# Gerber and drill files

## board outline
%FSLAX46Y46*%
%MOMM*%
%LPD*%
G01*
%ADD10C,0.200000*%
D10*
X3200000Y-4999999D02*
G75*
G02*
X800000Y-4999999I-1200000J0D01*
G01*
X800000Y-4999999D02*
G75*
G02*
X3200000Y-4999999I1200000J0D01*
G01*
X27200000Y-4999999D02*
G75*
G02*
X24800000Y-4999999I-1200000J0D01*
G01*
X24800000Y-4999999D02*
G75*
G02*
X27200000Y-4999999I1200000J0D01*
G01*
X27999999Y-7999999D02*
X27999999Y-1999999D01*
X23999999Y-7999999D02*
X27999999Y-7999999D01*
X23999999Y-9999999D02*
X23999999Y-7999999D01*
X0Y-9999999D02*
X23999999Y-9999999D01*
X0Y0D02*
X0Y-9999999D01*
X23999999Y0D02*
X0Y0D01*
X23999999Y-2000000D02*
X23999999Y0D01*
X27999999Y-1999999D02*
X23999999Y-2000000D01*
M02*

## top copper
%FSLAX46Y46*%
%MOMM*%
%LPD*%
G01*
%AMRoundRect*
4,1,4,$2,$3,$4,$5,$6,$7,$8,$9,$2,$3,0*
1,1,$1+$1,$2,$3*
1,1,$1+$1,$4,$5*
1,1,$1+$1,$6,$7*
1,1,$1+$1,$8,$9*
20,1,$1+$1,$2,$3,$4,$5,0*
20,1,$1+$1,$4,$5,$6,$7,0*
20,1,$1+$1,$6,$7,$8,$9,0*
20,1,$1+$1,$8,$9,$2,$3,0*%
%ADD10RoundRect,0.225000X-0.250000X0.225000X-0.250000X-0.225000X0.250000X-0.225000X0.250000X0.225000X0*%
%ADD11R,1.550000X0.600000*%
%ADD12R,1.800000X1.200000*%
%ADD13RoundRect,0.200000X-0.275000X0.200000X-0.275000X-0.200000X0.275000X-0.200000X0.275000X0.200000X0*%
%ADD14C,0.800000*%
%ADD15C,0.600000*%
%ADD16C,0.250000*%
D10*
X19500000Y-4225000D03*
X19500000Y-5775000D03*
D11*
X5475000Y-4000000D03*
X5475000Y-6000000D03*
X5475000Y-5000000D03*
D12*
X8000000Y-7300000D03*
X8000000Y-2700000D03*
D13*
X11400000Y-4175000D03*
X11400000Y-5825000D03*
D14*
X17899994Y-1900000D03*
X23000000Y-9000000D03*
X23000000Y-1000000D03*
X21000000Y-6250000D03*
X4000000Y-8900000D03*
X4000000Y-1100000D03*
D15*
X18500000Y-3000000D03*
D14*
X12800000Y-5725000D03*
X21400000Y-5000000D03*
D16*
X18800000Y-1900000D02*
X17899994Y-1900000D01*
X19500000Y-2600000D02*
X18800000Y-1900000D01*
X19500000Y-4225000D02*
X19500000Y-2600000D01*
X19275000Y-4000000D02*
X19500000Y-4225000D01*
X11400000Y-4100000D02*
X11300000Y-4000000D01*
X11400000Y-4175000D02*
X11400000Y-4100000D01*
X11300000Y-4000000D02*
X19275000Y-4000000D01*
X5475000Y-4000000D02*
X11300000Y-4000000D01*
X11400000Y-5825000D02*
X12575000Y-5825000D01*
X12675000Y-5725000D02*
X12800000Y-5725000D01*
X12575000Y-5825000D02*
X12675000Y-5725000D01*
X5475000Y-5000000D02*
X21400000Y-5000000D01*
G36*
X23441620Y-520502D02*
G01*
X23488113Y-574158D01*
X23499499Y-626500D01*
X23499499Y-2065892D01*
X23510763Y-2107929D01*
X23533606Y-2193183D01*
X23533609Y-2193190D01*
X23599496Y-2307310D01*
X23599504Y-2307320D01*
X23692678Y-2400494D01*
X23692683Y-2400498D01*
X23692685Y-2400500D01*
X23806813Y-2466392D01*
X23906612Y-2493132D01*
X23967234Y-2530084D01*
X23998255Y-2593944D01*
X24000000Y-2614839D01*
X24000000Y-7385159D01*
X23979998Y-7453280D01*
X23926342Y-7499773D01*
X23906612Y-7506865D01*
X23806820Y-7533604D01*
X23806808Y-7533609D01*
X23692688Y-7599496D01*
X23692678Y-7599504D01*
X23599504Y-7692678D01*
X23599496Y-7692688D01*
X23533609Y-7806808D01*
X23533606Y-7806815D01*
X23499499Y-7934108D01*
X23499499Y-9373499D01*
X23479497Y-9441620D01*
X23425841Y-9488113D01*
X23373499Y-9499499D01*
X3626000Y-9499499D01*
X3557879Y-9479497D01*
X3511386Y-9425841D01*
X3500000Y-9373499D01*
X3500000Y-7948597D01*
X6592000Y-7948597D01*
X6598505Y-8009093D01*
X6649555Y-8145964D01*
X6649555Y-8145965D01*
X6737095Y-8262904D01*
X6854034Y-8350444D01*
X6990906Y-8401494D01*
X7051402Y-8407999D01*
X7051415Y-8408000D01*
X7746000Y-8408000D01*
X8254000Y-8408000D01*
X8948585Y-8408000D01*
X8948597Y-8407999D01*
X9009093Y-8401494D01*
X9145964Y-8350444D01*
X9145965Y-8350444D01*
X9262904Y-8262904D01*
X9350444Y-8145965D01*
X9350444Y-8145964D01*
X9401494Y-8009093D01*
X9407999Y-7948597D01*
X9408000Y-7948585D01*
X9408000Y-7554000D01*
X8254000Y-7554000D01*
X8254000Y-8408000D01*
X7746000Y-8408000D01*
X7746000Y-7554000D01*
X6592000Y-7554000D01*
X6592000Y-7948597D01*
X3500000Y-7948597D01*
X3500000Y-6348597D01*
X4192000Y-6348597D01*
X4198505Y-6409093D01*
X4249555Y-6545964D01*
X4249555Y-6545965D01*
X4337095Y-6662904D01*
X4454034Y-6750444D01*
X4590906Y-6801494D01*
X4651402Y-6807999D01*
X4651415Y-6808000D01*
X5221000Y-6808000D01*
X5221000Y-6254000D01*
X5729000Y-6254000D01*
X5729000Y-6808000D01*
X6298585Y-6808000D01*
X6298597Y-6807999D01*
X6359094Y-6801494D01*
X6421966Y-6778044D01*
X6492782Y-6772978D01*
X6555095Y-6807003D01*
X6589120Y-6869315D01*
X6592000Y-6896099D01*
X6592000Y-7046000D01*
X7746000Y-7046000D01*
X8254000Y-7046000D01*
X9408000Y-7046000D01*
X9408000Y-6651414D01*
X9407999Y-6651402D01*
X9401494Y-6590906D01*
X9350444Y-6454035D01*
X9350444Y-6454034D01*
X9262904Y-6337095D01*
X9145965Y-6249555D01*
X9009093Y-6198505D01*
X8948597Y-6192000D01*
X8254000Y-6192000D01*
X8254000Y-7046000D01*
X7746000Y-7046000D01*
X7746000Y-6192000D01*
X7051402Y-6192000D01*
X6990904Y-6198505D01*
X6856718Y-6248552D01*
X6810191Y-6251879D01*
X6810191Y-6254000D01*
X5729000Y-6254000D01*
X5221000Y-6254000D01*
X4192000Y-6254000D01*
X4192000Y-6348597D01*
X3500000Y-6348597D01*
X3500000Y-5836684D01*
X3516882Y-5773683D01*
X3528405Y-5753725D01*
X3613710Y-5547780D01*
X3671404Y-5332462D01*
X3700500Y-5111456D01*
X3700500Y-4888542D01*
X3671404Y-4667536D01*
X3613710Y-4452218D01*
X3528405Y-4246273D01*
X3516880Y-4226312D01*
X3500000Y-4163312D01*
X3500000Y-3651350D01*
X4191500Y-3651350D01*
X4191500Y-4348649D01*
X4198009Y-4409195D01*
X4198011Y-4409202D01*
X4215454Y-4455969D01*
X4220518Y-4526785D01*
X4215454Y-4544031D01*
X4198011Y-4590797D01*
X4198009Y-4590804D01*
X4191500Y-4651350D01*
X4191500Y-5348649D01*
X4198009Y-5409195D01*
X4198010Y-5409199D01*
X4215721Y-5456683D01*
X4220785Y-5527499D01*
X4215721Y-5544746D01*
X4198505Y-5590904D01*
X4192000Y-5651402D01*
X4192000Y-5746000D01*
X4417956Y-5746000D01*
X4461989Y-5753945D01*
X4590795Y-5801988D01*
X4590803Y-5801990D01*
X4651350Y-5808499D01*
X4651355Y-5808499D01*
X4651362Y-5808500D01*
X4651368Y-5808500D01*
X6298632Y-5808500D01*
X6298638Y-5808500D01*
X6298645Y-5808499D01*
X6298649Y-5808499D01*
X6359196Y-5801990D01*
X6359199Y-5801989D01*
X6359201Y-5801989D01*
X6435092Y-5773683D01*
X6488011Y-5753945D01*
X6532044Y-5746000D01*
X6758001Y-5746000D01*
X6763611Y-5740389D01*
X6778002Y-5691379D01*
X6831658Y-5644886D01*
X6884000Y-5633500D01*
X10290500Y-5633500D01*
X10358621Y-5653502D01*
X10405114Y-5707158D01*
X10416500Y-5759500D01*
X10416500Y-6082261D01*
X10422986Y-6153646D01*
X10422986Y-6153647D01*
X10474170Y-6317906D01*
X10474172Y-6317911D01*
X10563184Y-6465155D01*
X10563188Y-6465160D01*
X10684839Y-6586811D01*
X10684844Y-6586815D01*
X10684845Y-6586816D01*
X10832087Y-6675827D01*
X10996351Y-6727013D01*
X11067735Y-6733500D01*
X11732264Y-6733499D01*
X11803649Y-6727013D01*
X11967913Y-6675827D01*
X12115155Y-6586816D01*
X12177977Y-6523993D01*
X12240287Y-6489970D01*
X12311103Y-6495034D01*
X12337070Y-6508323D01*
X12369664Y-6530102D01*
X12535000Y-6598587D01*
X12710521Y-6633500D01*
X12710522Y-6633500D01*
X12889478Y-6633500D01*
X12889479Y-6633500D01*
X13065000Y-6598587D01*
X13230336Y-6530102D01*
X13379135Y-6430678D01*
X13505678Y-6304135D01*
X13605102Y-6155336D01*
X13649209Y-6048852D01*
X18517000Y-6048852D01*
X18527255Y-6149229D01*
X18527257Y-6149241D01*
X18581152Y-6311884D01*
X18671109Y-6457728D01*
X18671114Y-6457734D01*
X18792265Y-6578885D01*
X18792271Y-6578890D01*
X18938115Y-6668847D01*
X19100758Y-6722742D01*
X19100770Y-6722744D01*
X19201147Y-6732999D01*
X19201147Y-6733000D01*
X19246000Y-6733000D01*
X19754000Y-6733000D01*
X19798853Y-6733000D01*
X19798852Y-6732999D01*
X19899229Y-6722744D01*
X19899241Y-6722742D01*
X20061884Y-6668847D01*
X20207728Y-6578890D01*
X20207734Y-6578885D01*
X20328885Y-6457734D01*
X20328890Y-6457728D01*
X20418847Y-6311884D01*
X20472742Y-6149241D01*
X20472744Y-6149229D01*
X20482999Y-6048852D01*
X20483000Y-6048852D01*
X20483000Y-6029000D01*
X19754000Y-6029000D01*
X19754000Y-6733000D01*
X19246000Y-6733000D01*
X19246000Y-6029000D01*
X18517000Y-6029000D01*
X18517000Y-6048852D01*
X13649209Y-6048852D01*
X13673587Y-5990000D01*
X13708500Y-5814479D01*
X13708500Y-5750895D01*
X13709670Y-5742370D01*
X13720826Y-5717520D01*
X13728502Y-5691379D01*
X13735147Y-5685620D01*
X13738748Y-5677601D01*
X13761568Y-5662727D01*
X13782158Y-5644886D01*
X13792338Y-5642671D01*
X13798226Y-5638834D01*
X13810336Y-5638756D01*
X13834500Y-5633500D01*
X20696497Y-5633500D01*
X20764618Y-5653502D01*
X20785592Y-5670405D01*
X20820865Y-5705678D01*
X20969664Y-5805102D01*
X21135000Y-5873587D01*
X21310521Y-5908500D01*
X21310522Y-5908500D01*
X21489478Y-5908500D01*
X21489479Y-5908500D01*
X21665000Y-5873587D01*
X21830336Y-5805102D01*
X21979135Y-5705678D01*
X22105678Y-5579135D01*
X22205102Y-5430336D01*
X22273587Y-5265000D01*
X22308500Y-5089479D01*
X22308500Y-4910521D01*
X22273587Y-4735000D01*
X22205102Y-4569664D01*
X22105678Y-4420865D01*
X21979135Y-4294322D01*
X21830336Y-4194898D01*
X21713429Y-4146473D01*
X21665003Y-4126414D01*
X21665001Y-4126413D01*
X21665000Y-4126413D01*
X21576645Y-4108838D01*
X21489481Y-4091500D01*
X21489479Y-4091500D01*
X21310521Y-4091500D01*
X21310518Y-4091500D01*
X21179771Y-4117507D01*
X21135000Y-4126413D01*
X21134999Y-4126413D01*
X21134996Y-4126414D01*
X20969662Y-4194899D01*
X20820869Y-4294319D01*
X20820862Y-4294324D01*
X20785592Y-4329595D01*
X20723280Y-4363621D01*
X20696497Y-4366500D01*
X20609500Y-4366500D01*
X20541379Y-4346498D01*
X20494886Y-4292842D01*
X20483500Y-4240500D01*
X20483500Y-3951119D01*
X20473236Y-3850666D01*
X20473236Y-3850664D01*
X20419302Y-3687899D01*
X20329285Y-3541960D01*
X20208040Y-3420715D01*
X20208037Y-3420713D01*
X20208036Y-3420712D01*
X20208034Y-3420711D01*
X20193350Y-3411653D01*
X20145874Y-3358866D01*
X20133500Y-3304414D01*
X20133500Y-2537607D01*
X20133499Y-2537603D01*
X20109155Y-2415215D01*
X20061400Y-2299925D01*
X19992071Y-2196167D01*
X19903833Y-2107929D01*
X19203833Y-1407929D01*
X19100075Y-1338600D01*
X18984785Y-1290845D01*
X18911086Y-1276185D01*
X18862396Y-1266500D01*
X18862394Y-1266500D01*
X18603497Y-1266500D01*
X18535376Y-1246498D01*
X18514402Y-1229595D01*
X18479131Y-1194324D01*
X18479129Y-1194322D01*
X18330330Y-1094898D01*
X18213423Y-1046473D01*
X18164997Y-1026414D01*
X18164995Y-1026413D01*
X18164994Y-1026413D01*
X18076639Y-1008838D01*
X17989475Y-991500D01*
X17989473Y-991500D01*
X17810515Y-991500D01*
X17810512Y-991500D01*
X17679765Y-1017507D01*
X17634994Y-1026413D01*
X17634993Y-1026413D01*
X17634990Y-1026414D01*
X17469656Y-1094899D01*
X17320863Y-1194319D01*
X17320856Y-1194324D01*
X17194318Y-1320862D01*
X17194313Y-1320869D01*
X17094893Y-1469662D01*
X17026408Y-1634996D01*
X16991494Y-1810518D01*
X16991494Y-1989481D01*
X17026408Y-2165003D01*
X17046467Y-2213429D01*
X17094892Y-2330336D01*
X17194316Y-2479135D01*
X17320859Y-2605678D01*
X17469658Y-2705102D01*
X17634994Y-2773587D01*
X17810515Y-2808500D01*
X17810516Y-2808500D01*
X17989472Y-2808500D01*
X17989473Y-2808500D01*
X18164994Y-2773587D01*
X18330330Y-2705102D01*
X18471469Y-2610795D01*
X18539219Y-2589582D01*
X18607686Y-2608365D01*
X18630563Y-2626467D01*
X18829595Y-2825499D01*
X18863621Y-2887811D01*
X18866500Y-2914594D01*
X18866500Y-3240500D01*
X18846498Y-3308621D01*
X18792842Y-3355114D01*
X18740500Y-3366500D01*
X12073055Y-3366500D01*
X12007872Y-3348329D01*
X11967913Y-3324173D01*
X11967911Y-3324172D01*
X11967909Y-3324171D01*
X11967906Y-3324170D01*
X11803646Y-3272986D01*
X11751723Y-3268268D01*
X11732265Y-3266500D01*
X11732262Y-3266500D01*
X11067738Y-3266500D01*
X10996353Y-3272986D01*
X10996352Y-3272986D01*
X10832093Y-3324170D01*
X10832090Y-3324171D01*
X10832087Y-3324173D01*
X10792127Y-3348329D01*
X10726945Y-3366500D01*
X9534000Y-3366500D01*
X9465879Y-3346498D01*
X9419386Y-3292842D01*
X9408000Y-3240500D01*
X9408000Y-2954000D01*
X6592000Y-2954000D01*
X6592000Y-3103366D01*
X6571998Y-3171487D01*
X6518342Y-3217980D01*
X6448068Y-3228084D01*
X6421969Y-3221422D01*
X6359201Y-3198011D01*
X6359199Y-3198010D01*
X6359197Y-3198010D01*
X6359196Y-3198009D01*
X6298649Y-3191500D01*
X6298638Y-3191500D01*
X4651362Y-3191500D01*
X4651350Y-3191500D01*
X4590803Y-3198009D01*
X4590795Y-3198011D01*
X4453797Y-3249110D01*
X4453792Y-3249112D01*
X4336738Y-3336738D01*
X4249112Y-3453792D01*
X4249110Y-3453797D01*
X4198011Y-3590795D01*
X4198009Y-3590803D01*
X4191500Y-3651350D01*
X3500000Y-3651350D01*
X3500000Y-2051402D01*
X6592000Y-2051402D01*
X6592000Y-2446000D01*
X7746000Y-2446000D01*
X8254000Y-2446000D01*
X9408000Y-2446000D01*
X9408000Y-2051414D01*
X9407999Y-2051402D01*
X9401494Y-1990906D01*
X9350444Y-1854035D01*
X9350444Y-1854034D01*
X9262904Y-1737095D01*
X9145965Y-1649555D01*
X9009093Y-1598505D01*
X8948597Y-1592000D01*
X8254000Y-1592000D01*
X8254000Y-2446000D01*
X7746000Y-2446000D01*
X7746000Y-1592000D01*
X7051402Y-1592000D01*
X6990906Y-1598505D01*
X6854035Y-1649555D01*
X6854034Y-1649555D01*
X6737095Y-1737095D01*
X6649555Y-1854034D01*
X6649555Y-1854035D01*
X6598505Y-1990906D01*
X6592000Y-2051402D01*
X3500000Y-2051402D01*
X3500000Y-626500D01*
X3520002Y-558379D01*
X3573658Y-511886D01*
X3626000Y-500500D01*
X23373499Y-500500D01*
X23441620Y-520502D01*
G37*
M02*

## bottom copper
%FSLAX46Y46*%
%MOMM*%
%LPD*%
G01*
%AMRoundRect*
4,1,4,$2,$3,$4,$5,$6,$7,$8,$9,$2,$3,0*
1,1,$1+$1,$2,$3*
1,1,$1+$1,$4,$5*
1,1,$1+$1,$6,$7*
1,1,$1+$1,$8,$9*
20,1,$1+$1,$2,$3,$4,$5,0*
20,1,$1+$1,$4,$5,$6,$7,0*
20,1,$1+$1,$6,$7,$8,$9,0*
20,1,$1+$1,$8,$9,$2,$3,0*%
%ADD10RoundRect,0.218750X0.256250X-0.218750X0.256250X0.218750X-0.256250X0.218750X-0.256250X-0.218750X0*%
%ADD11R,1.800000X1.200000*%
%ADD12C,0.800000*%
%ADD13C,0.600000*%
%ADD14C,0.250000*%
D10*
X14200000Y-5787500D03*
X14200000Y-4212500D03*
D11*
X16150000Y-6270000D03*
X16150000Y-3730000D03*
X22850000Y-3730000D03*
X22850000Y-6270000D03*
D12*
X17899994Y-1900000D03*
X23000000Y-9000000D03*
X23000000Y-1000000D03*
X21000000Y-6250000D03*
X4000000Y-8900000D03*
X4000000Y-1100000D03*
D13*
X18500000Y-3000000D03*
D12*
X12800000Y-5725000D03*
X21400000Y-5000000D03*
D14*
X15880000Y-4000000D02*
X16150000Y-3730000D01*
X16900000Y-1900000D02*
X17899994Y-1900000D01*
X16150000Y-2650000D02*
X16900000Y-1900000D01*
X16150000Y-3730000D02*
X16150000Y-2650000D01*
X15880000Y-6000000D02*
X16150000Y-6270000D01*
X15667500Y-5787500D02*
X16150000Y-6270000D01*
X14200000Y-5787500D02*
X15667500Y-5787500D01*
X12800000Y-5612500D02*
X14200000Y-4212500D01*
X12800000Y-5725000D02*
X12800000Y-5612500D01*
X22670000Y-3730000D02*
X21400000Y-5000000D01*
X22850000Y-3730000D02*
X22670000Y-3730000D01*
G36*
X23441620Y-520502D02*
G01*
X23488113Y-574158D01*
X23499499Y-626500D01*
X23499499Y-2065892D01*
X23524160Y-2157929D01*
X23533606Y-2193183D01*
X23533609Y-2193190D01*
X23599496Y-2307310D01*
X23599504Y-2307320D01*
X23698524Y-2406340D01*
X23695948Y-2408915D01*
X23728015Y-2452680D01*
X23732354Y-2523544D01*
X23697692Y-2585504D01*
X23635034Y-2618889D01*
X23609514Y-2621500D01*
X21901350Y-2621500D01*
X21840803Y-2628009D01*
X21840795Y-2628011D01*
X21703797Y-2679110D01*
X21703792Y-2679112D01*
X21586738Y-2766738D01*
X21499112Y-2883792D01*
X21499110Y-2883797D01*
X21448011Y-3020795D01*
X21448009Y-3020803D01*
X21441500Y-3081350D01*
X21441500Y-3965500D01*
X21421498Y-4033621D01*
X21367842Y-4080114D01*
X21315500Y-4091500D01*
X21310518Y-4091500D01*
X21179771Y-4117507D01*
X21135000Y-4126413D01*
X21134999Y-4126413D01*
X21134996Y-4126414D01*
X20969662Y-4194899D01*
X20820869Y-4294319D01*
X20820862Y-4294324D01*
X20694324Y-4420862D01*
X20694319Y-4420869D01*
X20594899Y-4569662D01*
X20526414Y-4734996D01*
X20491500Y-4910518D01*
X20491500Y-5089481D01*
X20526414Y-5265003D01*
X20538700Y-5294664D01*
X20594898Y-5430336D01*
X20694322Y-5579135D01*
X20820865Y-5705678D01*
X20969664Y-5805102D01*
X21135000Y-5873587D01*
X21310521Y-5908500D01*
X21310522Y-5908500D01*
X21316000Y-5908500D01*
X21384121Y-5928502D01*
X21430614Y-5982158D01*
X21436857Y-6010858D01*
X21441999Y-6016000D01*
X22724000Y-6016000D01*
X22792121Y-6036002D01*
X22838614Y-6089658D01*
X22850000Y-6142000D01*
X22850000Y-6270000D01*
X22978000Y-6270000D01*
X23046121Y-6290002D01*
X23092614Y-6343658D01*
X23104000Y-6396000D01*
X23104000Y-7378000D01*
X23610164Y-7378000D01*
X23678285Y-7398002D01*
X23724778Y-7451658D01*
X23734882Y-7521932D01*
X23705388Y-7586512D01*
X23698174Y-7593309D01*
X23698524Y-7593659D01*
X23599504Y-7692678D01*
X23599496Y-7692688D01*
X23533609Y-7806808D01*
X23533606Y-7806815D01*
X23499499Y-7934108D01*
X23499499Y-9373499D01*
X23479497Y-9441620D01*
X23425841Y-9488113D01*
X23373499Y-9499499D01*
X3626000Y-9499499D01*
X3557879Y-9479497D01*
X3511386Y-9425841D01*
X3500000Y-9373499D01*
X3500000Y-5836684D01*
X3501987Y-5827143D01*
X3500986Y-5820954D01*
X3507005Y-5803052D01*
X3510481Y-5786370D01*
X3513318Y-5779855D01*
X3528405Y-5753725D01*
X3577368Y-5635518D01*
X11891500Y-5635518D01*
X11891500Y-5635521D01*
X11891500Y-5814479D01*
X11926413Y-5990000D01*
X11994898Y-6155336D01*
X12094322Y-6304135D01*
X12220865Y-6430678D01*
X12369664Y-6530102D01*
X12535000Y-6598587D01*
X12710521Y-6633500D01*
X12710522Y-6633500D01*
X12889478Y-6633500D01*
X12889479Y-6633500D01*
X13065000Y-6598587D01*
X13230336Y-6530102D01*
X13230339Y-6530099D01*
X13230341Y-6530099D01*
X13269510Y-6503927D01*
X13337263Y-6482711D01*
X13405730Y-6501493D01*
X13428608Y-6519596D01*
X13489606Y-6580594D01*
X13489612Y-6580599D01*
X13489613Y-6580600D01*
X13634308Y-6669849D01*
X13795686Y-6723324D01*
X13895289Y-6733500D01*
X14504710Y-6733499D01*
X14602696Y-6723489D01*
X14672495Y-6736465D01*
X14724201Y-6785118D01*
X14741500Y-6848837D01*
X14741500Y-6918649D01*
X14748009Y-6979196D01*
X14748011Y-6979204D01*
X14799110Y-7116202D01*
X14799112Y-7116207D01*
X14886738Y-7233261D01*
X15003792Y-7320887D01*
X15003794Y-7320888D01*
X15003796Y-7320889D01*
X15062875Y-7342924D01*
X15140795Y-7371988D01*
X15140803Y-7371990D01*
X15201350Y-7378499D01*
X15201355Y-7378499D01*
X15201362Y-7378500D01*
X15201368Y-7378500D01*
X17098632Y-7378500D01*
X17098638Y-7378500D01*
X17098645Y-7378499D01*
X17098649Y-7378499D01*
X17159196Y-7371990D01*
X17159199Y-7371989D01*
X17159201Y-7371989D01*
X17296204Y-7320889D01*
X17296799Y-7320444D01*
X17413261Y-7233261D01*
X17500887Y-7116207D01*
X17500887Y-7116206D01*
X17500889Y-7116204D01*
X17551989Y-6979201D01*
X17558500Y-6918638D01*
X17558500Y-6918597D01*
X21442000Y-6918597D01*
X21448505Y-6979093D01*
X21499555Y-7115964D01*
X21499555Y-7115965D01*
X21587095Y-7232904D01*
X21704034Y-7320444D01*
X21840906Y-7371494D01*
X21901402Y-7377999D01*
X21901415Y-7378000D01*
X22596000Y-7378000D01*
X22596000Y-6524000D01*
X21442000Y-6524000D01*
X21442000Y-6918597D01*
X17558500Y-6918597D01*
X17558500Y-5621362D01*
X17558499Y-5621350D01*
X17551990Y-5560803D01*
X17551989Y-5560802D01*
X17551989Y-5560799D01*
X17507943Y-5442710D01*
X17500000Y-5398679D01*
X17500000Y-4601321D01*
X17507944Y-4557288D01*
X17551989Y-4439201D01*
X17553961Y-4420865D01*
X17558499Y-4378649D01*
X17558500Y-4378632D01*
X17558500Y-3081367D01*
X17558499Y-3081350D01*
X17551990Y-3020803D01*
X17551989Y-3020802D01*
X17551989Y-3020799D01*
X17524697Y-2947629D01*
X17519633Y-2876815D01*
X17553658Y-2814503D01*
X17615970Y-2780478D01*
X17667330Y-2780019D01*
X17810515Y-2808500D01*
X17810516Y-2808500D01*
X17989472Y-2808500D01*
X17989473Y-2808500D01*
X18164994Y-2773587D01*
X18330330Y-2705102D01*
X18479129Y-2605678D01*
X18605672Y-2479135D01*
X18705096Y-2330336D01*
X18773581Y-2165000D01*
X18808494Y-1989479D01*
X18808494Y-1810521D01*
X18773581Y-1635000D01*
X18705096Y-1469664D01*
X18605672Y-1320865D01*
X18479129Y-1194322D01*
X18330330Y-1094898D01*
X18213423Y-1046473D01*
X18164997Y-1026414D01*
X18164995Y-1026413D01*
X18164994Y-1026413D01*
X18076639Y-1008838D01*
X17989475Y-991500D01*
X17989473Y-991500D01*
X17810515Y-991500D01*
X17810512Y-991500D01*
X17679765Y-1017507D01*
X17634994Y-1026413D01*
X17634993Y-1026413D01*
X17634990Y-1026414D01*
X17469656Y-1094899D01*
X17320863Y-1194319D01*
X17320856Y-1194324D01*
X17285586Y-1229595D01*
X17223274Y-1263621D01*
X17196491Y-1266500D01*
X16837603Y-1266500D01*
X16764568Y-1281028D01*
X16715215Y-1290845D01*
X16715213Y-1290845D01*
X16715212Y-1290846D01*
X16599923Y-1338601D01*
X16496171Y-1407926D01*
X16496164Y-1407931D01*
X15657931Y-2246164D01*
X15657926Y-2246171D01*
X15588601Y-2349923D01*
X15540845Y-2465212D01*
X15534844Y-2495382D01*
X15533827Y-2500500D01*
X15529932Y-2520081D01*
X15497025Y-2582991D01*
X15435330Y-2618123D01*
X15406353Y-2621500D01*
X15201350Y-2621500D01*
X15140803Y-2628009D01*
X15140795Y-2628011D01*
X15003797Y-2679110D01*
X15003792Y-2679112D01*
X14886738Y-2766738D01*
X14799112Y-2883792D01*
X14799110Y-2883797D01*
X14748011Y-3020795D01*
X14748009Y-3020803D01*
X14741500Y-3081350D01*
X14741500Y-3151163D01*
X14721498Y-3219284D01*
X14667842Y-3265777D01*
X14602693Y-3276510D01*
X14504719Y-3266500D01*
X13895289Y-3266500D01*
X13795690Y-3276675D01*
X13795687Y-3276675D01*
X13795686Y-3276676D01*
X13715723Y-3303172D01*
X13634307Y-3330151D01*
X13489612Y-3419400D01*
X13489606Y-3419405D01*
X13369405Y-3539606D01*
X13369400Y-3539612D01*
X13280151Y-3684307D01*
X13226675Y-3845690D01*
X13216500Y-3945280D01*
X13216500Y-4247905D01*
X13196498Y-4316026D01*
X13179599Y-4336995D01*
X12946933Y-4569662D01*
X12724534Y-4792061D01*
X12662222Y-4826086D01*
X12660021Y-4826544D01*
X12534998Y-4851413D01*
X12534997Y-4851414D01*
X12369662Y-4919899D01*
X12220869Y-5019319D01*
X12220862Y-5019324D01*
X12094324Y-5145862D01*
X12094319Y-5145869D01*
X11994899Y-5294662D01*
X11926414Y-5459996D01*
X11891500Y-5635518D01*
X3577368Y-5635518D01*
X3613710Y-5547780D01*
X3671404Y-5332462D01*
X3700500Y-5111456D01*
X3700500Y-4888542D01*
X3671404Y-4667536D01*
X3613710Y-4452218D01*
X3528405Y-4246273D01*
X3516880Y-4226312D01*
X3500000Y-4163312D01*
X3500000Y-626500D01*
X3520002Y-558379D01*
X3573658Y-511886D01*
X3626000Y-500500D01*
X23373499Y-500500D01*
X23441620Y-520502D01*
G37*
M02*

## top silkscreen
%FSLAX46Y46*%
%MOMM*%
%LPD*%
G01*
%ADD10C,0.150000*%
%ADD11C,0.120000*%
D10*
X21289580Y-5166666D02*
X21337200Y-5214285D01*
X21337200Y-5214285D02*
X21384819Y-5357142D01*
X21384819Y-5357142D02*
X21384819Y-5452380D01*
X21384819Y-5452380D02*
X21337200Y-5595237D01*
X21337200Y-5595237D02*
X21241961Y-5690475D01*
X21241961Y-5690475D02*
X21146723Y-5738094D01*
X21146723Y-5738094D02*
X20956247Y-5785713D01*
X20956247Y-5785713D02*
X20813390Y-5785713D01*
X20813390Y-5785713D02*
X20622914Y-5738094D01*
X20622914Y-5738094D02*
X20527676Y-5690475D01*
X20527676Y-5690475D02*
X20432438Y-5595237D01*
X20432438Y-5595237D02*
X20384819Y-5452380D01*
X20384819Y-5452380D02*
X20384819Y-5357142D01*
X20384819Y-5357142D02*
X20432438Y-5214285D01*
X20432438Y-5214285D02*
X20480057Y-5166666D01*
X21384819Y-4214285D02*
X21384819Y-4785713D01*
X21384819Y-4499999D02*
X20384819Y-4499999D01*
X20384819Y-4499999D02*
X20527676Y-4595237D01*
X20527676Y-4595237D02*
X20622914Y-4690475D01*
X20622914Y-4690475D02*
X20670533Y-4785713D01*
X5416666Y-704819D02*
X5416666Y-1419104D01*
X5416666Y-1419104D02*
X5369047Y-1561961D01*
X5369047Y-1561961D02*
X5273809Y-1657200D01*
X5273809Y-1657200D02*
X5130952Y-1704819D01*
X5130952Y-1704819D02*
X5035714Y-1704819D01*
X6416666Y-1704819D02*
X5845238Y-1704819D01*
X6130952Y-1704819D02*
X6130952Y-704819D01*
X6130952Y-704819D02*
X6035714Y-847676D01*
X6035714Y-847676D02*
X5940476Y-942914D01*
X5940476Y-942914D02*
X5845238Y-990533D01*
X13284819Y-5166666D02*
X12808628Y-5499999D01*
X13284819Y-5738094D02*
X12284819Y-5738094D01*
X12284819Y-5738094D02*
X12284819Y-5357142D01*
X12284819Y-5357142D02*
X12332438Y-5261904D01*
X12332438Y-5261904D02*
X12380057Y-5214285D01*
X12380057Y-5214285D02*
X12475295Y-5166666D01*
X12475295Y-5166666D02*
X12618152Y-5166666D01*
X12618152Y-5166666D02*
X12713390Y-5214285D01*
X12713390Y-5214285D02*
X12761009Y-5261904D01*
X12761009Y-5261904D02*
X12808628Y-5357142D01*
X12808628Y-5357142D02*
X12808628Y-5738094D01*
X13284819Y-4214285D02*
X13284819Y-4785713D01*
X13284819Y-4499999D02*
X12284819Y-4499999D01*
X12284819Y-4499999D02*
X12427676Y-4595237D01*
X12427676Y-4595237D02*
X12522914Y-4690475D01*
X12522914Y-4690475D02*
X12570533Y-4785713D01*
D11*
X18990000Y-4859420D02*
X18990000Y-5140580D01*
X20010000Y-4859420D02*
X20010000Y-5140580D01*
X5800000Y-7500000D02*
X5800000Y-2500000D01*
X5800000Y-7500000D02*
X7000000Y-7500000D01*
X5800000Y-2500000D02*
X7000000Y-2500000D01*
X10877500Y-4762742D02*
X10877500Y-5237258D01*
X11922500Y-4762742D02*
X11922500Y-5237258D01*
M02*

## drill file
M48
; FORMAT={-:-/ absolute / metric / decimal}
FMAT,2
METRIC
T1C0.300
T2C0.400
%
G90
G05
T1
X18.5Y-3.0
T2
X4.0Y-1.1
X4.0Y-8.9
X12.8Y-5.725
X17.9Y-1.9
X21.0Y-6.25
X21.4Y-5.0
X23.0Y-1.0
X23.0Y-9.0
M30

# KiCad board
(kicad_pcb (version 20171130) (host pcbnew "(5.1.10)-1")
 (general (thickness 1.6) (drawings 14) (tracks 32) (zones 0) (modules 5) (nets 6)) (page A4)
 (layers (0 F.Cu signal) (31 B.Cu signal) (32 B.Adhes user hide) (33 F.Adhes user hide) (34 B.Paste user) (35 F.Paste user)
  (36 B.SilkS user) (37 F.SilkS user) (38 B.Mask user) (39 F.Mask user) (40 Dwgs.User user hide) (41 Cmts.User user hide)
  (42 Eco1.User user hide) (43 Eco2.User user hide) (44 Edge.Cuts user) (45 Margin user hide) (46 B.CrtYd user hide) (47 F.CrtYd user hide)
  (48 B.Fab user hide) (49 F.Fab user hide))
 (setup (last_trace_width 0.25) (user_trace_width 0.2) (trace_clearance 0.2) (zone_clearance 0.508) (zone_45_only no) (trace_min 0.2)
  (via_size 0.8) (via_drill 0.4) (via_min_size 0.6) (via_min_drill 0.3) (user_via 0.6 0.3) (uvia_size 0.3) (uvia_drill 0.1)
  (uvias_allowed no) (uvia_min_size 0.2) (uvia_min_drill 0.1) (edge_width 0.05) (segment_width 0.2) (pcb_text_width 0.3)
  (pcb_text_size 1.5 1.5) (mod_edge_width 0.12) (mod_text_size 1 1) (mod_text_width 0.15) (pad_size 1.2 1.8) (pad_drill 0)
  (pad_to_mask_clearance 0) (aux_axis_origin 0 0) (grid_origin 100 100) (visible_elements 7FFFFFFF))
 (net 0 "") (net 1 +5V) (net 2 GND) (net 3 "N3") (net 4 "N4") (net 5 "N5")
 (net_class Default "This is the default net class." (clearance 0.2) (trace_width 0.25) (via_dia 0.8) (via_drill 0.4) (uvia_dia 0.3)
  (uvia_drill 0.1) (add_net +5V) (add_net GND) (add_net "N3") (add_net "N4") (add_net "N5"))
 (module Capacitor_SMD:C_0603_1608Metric (layer F.Cu) (at 19.5 5 270)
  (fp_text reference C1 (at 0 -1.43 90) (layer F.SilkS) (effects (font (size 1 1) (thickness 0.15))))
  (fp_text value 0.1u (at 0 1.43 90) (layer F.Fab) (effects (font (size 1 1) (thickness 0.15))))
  (fp_line (start -0.14058 0.51) (end 0.14058 0.51) (layer F.SilkS) (width 0.12))
  (fp_line (start -0.14058 -0.51) (end 0.14058 -0.51) (layer F.SilkS) (width 0.12))
  (pad 1 smd roundrect (at -0.775 0 270) (size 0.9 0.95) (layers F.Cu F.Paste F.Mask) (roundrect_rratio 0.25) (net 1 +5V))
  (pad 2 smd roundrect (at 0.775 0 270) (size 0.9 0.95) (layers F.Cu F.Paste F.Mask) (roundrect_rratio 0.25) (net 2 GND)))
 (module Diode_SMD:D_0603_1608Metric (layer B.Cu) (at 14.2 5 90)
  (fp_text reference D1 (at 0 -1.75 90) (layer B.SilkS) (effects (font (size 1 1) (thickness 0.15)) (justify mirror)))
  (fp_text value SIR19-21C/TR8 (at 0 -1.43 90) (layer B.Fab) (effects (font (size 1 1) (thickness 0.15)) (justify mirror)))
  (pad 1 smd roundrect (at -0.7875 0 90) (size 0.875 0.95) (layers B.Cu B.Paste B.Mask) (roundrect_rratio 0.25) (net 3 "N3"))
  (pad 2 smd roundrect (at 0.7875 0 90) (size 0.875 0.95) (layers B.Cu B.Paste B.Mask) (roundrect_rratio 0.25) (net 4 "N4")))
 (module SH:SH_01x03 (layer F.Cu) (at 8 5 90)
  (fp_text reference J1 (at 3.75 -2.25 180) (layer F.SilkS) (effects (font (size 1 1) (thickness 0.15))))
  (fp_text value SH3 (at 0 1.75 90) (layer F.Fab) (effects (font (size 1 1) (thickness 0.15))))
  (fp_line (start -2.5 -2.2) (end 2.5 -2.2) (layer F.SilkS) (width 0.12))
  (fp_line (start -2.5 -2.2) (end -2.5 -1) (layer F.SilkS) (width 0.12))
  (fp_line (start 2.5 -2.2) (end 2.5 -1) (layer F.SilkS) (width 0.12))
  (pad 3 smd rect (at 1 -2.525 90) (size 0.6 1.55) (layers F.Cu F.Paste F.Mask) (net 1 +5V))
  (pad 1 smd rect (at -1 -2.525 90) (size 0.6 1.55) (layers F.Cu F.Paste F.Mask) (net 2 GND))
  (pad 2 smd rect (at 0 -2.525 90) (size 0.6 1.55) (layers F.Cu F.Paste F.Mask) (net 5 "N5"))
  (pad MP smd rect (at -2.3 0 90) (size 1.2 1.8) (layers F.Cu F.Paste F.Mask) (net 2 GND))
  (pad MP smd rect (at 2.3 0 90) (size 1.2 1.8) (layers F.Cu F.Paste F.Mask) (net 2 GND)))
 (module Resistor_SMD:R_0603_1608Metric (layer F.Cu) (at 11.4 5 270)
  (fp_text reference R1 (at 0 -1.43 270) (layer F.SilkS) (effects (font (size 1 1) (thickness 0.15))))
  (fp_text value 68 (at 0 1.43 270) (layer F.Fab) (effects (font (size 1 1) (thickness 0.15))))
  (fp_line (start -0.237258 0.5225) (end 0.237258 0.5225) (layer F.SilkS) (width 0.12))
  (fp_line (start -0.237258 -0.5225) (end 0.237258 -0.5225) (layer F.SilkS) (width 0.12))
  (pad 1 smd roundrect (at -0.825 0 270) (size 0.8 0.95) (layers F.Cu F.Paste F.Mask) (roundrect_rratio 0.25) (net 1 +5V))
  (pad 2 smd roundrect (at 0.825 0 270) (size 0.8 0.95) (layers F.Cu F.Paste F.Mask) (roundrect_rratio 0.25) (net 4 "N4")))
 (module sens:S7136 (layer B.Cu) (at 19.5 5)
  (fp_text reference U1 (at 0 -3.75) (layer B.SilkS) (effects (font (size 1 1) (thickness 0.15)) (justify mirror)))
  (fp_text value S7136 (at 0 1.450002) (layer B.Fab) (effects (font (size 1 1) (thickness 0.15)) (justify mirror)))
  (pad 1 smd rect (at -3.35 1.27) (size 1.8 1.2) (layers B.Cu B.Paste B.Mask) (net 3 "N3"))
  (pad 2 smd rect (at -3.35 -1.27) (size 1.8 1.2) (layers B.Cu B.Paste B.Mask) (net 1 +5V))
  (pad 3 smd rect (at 3.35 -1.27) (size 1.8 1.2) (layers B.Cu B.Paste B.Mask) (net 5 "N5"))
  (pad 4 smd rect (at 3.35 1.27) (size 1.8 1.2) (layers B.Cu B.Paste B.Mask) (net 2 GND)))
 (gr_circle (center 2 4.999999) (end 3.2 4.999999) (layer Edge.Cuts) (width 0.2))
 (gr_circle (center 26 4.999999) (end 27.2 4.999999) (layer Edge.Cuts) (width 0.2))
 (gr_line (start 27.999999 7.999999) (end 27.999999 1.999999) (layer Edge.Cuts) (width 0.2))
 (gr_line (start 23.999999 7.999999) (end 27.999999 7.999999) (layer Edge.Cuts) (width 0.2))
 (gr_line (start 23.999999 9.999999) (end 23.999999 7.999999) (layer Edge.Cuts) (width 0.2))
 (gr_line (start 0 9.999999) (end 23.999999 9.999999) (layer Edge.Cuts) (width 0.2))
 (gr_line (start 0 0) (end 0 9.999999) (layer Edge.Cuts) (width 0.2))
 (gr_line (start 23.999999 0) (end 0 0) (layer Edge.Cuts) (width 0.2))
 (gr_line (start 23.999999 2) (end 23.999999 0) (layer Edge.Cuts) (width 0.2))
 (gr_line (start 27.999999 1.999999) (end 23.999999 2) (layer Edge.Cuts) (width 0.2))
 (segment (start 15.88 4) (end 16.15 3.73) (width 0.25) (layer B.Cu) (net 1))
 (via (at 17.899994 1.9) (size 0.8) (drill 0.4) (layers F.Cu B.Cu) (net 1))
 (segment (start 16.9 1.9) (end 17.899994 1.9) (width 0.25) (layer B.Cu) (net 1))
 (segment (start 16.15 2.65) (end 16.9 1.9) (width 0.25) (layer B.Cu) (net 1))
 (segment (start 16.15 3.73) (end 16.15 2.65) (width 0.25) (layer B.Cu) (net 1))
 (segment (start 18.8 1.9) (end 17.899994 1.9) (width 0.25) (layer F.Cu) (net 1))
 (segment (start 19.5 2.6) (end 18.8 1.9) (width 0.25) (layer F.Cu) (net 1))
 (segment (start 19.5 4.225) (end 19.5 2.6) (width 0.25) (layer F.Cu) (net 1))
 (segment (start 19.275 4) (end 19.5 4.225) (width 0.25) (layer F.Cu) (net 1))
 (segment (start 11.4 4.1) (end 11.3 4) (width 0.25) (layer F.Cu) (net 1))
 (segment (start 11.4 4.175) (end 11.4 4.1) (width 0.25) (layer F.Cu) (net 1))
 (segment (start 11.3 4) (end 19.275 4) (width 0.25) (layer F.Cu) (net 1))
 (segment (start 5.475 4) (end 11.3 4) (width 0.25) (layer F.Cu) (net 1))
 (via (at 23 9) (size 0.8) (drill 0.4) (layers F.Cu B.Cu) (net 2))
 (via (at 23 1) (size 0.8) (drill 0.4) (layers F.Cu B.Cu) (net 2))
 (via (at 21 6.25) (size 0.8) (drill 0.4) (layers F.Cu B.Cu) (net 2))
 (via (at 4 8.9) (size 0.8) (drill 0.4) (layers F.Cu B.Cu) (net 2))
 (via (at 4 1.1) (size 0.8) (drill 0.4) (layers F.Cu B.Cu) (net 2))
 (via (at 18.5 3) (size 0.6) (drill 0.3) (layers F.Cu B.Cu) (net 2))
 (segment (start 15.88 6) (end 16.15 6.27) (width 0.25) (layer B.Cu) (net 3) (status 30))
 (segment (start 15.6675 5.7875) (end 16.15 6.27) (width 0.25) (layer B.Cu) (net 3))
 (segment (start 14.2 5.7875) (end 15.6675 5.7875) (width 0.25) (layer B.Cu) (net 3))
 (segment (start 11.4 5.825) (end 12.575 5.825) (width 0.25) (layer F.Cu) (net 4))
 (segment (start 12.675 5.725) (end 12.8 5.725) (width 0.25) (layer F.Cu) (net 4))
 (via (at 12.8 5.725) (size 0.8) (drill 0.4) (layers F.Cu B.Cu) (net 4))
 (segment (start 12.575 5.825) (end 12.675 5.725) (width 0.25) (layer F.Cu) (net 4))
 (segment (start 12.8 5.6125) (end 14.2 4.2125) (width 0.25) (layer B.Cu) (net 4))
 (segment (start 12.8 5.725) (end 12.8 5.6125) (width 0.25) (layer B.Cu) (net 4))
 (segment (start 22.67 3.73) (end 21.4 5) (width 0.25) (layer B.Cu) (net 5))
 (segment (start 22.85 3.73) (end 22.67 3.73) (width 0.25) (layer B.Cu) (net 5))
 (segment (start 5.475 5) (end 21.4 5) (width 0.25) (layer F.Cu) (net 5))
 (via (at 21.4 5) (size 0.8) (drill 0.4) (layers F.Cu B.Cu) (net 5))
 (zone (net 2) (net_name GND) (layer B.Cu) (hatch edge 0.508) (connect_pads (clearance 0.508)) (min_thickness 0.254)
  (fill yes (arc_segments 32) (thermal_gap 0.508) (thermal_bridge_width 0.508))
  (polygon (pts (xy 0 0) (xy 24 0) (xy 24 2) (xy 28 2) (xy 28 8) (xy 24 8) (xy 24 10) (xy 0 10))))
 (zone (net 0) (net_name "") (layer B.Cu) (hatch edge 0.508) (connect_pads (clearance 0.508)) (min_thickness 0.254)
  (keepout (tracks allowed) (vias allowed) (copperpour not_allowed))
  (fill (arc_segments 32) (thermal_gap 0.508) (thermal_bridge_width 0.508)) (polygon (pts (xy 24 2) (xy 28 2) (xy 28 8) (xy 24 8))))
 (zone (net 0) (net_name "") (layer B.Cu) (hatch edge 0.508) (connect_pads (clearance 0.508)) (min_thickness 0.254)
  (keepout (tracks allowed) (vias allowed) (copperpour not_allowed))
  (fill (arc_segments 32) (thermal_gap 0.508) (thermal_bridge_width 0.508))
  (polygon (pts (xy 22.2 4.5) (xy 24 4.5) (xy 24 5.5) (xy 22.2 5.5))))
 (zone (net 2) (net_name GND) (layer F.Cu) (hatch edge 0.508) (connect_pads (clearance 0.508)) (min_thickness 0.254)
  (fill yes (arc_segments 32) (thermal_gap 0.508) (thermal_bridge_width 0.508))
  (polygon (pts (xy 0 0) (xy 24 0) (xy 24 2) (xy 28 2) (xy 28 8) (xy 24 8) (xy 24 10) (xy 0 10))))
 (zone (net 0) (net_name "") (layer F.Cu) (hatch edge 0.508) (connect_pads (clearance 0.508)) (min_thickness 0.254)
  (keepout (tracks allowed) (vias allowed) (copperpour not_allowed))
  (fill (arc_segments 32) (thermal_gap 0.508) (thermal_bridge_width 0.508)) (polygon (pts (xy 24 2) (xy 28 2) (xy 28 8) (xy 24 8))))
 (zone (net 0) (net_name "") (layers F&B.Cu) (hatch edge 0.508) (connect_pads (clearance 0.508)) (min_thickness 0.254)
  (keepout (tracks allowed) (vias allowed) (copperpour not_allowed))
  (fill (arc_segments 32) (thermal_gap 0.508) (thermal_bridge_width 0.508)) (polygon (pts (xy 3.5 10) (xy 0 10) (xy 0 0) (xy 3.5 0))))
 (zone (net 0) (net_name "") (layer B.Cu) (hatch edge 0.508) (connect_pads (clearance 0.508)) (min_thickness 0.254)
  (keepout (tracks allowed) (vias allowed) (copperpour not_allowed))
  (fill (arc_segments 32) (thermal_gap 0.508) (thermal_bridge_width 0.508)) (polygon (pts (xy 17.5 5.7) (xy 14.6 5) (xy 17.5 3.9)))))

